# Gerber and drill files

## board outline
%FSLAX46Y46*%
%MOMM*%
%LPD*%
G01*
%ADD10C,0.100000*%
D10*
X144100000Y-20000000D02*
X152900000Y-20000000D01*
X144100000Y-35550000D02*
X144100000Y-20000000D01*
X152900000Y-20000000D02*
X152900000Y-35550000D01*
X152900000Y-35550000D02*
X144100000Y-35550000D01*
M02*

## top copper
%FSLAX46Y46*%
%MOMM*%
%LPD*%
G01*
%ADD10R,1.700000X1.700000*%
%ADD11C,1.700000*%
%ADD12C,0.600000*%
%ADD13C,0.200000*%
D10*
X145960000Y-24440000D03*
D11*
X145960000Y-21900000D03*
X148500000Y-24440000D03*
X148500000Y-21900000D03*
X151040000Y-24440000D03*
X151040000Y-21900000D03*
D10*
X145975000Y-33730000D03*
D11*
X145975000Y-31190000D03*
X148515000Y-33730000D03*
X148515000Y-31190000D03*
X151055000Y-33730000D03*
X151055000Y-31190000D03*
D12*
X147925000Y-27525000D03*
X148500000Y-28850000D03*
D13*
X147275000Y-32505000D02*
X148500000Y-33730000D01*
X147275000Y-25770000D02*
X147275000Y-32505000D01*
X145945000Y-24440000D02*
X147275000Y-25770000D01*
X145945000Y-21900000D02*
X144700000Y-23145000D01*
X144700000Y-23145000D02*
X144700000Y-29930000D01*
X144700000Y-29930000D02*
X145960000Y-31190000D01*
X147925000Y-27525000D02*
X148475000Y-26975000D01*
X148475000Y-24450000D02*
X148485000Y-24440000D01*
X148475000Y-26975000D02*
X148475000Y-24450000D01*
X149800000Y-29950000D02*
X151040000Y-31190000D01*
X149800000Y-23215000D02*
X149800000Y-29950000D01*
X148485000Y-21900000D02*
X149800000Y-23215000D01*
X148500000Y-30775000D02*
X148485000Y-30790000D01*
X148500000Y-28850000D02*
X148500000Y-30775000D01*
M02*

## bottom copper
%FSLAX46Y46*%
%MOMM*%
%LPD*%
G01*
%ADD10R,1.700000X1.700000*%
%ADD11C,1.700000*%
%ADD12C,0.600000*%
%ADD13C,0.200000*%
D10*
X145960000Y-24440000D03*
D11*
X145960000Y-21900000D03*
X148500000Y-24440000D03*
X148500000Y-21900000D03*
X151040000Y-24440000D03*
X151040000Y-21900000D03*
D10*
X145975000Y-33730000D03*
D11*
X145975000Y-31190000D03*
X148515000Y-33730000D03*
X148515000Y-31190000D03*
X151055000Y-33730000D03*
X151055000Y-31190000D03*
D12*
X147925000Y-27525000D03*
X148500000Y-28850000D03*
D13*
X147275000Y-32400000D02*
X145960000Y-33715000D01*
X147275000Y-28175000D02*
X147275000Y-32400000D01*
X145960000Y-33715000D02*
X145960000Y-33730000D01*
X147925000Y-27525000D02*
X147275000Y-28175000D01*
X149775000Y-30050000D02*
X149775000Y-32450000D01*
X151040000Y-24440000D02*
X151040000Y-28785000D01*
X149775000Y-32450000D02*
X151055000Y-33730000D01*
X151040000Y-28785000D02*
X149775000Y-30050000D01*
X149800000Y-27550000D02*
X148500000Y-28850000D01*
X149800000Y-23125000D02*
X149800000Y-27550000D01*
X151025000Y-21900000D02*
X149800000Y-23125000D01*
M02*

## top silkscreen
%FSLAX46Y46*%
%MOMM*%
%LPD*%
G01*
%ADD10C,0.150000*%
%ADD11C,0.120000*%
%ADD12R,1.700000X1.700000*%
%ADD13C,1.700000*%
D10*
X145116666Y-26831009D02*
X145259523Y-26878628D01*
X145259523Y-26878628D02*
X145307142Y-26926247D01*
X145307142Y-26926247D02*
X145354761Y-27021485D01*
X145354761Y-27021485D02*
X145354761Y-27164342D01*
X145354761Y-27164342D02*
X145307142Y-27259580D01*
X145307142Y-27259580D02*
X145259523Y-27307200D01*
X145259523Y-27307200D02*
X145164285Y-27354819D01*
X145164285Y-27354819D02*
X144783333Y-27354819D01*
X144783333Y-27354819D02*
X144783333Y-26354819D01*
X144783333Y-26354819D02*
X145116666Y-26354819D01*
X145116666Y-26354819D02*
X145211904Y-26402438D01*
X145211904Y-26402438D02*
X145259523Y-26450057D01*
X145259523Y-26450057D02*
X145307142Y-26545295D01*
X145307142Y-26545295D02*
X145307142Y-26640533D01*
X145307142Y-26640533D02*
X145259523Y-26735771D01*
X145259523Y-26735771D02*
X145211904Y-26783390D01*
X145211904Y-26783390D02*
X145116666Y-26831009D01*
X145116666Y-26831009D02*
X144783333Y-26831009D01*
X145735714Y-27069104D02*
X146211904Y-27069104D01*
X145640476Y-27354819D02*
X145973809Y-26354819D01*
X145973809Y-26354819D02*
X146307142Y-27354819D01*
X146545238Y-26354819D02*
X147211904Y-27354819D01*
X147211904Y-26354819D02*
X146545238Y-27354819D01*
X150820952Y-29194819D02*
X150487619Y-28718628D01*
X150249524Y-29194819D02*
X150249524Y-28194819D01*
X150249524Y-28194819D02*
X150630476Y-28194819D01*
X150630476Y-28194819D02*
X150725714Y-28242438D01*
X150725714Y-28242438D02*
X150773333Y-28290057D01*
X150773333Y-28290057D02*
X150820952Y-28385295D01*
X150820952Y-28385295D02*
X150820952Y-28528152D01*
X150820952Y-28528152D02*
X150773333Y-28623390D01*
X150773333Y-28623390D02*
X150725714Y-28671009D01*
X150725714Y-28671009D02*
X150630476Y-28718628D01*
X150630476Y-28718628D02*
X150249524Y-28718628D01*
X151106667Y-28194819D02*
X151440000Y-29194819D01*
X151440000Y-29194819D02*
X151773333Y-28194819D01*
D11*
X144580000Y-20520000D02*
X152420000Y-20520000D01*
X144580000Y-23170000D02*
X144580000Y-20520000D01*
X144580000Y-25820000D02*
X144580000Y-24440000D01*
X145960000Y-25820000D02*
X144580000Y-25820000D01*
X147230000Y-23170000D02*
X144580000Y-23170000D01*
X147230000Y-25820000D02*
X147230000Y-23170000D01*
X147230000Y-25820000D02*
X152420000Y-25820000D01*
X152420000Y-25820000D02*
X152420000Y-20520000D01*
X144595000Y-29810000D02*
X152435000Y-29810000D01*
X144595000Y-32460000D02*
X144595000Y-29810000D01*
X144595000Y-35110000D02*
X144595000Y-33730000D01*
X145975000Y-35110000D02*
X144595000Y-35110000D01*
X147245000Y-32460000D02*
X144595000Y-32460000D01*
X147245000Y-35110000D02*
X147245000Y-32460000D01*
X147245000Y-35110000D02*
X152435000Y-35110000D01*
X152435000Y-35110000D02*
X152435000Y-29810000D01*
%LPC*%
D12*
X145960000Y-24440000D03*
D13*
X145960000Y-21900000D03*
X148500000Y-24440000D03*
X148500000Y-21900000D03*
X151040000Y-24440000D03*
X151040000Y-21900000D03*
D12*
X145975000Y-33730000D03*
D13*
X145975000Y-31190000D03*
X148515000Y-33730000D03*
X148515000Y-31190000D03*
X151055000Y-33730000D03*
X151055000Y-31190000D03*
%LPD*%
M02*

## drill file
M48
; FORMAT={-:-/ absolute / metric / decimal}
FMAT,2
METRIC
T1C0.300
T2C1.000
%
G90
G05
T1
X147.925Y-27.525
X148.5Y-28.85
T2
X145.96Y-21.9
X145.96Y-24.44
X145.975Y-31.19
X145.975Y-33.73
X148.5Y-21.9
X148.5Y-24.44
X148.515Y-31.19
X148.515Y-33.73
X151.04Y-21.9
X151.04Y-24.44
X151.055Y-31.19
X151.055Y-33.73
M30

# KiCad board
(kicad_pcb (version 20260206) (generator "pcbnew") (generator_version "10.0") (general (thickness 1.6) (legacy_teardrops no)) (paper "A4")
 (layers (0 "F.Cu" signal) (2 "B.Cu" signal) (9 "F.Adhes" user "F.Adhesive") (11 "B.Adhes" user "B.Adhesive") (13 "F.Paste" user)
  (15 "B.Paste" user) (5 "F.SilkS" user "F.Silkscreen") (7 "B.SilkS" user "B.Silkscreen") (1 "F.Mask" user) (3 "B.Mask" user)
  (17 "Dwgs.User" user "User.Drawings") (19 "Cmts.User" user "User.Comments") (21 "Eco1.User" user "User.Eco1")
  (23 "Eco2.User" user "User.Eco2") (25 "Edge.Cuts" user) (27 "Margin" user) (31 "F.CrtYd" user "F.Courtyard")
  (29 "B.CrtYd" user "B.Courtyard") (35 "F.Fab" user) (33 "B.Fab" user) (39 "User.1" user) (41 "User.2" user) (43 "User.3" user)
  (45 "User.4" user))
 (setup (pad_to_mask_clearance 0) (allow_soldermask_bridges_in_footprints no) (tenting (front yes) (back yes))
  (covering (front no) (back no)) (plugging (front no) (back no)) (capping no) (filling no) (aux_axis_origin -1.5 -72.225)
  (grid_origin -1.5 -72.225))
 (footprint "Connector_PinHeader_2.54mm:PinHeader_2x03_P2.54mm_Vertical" (layer "F.Cu") (at 145.96 24.44 90)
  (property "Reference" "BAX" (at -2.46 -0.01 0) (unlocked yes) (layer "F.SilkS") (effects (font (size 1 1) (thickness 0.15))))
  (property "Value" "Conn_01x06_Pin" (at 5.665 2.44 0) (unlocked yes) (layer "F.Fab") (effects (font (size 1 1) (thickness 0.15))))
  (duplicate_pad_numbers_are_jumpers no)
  (fp_line (start 3.92 -1.38) (end 3.92 6.46) (stroke (width 0.12) (type solid)) (layer "F.SilkS"))
  (fp_line (start 1.27 -1.38) (end 3.92 -1.38) (stroke (width 0.12) (type solid)) (layer "F.SilkS"))
  (fp_line (start -1.38 -1.38) (end 0 -1.38) (stroke (width 0.12) (type solid)) (layer "F.SilkS"))
  (fp_line (start -1.38 0) (end -1.38 -1.38) (stroke (width 0.12) (type solid)) (layer "F.SilkS"))
  (fp_line (start 1.27 1.27) (end 1.27 -1.38) (stroke (width 0.12) (type solid)) (layer "F.SilkS"))
  (fp_line (start -1.38 1.27) (end 1.27 1.27) (stroke (width 0.12) (type solid)) (layer "F.SilkS"))
  (fp_line (start -1.38 1.27) (end -1.38 6.46) (stroke (width 0.12) (type solid)) (layer "F.SilkS"))
  (fp_line (start -1.38 6.46) (end 3.92 6.46) (stroke (width 0.12) (type solid)) (layer "F.SilkS"))
  (pad "1" thru_hole rect (at 0 0 90) (size 1.7 1.7) (drill 1) (layers "*.Cu" "*.Mask") (remove_unused_layers no) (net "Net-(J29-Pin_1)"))
  (pad "2" thru_hole circle (at 2.54 0 90) (size 1.7 1.7) (drill 1) (layers "*.Cu" "*.Mask") (remove_unused_layers no)
   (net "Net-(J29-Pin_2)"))
  (pad "3" thru_hole circle (at 0 2.54 90) (size 1.7 1.7) (drill 1) (layers "*.Cu" "*.Mask") (remove_unused_layers no)
   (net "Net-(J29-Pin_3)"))
  (pad "4" thru_hole circle (at 2.54 2.54 90) (size 1.7 1.7) (drill 1) (layers "*.Cu" "*.Mask") (remove_unused_layers no)
   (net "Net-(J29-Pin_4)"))
  (pad "5" thru_hole circle (at 0 5.08 90) (size 1.7 1.7) (drill 1) (layers "*.Cu" "*.Mask") (remove_unused_layers no)
   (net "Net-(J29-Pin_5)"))
  (pad "6" thru_hole circle (at 2.54 5.08 90) (size 1.7 1.7) (drill 1) (layers "*.Cu" "*.Mask") (remove_unused_layers no)
   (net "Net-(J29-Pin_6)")))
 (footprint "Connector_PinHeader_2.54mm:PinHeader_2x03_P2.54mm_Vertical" (layer "F.Cu") (at 145.975 33.73 90)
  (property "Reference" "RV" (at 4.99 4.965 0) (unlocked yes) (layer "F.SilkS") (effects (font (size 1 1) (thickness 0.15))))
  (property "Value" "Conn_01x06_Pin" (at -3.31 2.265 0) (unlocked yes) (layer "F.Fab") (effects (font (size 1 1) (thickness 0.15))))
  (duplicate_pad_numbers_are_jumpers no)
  (fp_line (start 3.92 -1.38) (end 3.92 6.46) (stroke (width 0.12) (type solid)) (layer "F.SilkS"))
  (fp_line (start 1.27 -1.38) (end 3.92 -1.38) (stroke (width 0.12) (type solid)) (layer "F.SilkS"))
  (fp_line (start -1.38 -1.38) (end 0 -1.38) (stroke (width 0.12) (type solid)) (layer "F.SilkS"))
  (fp_line (start -1.38 0) (end -1.38 -1.38) (stroke (width 0.12) (type solid)) (layer "F.SilkS"))
  (fp_line (start 1.27 1.27) (end 1.27 -1.38) (stroke (width 0.12) (type solid)) (layer "F.SilkS"))
  (fp_line (start -1.38 1.27) (end 1.27 1.27) (stroke (width 0.12) (type solid)) (layer "F.SilkS"))
  (fp_line (start -1.38 1.27) (end -1.38 6.46) (stroke (width 0.12) (type solid)) (layer "F.SilkS"))
  (fp_line (start -1.38 6.46) (end 3.92 6.46) (stroke (width 0.12) (type solid)) (layer "F.SilkS"))
  (pad "1" thru_hole rect (at 0 0 90) (size 1.7 1.7) (drill 1) (layers "*.Cu" "*.Mask") (remove_unused_layers no) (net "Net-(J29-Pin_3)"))
  (pad "2" thru_hole circle (at 2.54 0 90) (size 1.7 1.7) (drill 1) (layers "*.Cu" "*.Mask") (remove_unused_layers no)
   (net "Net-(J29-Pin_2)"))
  (pad "3" thru_hole circle (at 0 2.54 90) (size 1.7 1.7) (drill 1) (layers "*.Cu" "*.Mask") (remove_unused_layers no)
   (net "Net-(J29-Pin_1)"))
  (pad "4" thru_hole circle (at 2.54 2.54 90) (size 1.7 1.7) (drill 1) (layers "*.Cu" "*.Mask") (remove_unused_layers no)
   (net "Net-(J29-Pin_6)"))
  (pad "5" thru_hole circle (at 0 5.08 90) (size 1.7 1.7) (drill 1) (layers "*.Cu" "*.Mask") (remove_unused_layers no)
   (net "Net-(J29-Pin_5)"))
  (pad "6" thru_hole circle (at 2.54 5.08 90) (size 1.7 1.7) (drill 1) (layers "*.Cu" "*.Mask") (remove_unused_layers no)
   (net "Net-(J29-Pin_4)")))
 (gr_line (start 144.1 20) (end 152.9 20) (stroke (width 0.1) (type default)) (layer "Edge.Cuts"))
 (gr_line (start 144.1 35.55) (end 144.1 20) (stroke (width 0.1) (type default)) (layer "Edge.Cuts"))
 (gr_line (start 152.9 20) (end 152.9 35.55) (stroke (width 0.1) (type default)) (layer "Edge.Cuts"))
 (gr_line (start 152.9 35.55) (end 144.1 35.55) (stroke (width 0.1) (type default)) (layer "Edge.Cuts"))
 (segment (start 147.275 32.505) (end 148.5 33.73) (width 0.2) (layer "F.Cu") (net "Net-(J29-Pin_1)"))
 (segment (start 147.275 25.77) (end 147.275 32.505) (width 0.2) (layer "F.Cu") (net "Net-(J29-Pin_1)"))
 (segment (start 145.945 24.44) (end 147.275 25.77) (width 0.2) (layer "F.Cu") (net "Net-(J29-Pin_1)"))
 (segment (start 145.945 21.9) (end 144.7 23.145) (width 0.2) (layer "F.Cu") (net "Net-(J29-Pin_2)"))
 (segment (start 144.7 23.145) (end 144.7 29.93) (width 0.2) (layer "F.Cu") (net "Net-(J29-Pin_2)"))
 (segment (start 144.7 29.93) (end 145.96 31.19) (width 0.2) (layer "F.Cu") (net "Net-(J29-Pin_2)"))
 (segment (start 147.925 27.525) (end 148.475 26.975) (width 0.2) (layer "F.Cu") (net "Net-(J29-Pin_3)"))
 (segment (start 148.475 24.45) (end 148.485 24.44) (width 0.2) (layer "F.Cu") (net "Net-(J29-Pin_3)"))
 (segment (start 148.475 26.975) (end 148.475 24.45) (width 0.2) (layer "F.Cu") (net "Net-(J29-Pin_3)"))
 (via (at 147.925 27.525) (size 0.6) (drill 0.3) (layers "F.Cu" "B.Cu") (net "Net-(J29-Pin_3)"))
 (segment (start 147.275 32.4) (end 145.96 33.715) (width 0.2) (layer "B.Cu") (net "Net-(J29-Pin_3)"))
 (segment (start 147.275 28.175) (end 147.275 32.4) (width 0.2) (layer "B.Cu") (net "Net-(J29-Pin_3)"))
 (segment (start 145.96 33.715) (end 145.96 33.73) (width 0.2) (layer "B.Cu") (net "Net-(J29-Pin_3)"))
 (segment (start 147.925 27.525) (end 147.275 28.175) (width 0.2) (layer "B.Cu") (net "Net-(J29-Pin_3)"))
 (segment (start 149.8 29.95) (end 151.04 31.19) (width 0.2) (layer "F.Cu") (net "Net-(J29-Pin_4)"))
 (segment (start 149.8 23.215) (end 149.8 29.95) (width 0.2) (layer "F.Cu") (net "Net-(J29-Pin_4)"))
 (segment (start 148.485 21.9) (end 149.8 23.215) (width 0.2) (layer "F.Cu") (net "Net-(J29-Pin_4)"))
 (segment (start 149.775 30.05) (end 149.775 32.45) (width 0.2) (layer "B.Cu") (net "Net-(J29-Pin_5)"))
 (segment (start 151.04 24.44) (end 151.04 28.785) (width 0.2) (layer "B.Cu") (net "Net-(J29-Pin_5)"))
 (segment (start 149.775 32.45) (end 151.055 33.73) (width 0.2) (layer "B.Cu") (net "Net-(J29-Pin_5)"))
 (segment (start 151.04 28.785) (end 149.775 30.05) (width 0.2) (layer "B.Cu") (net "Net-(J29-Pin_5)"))
 (segment (start 148.5 30.775) (end 148.485 30.79) (width 0.2) (layer "F.Cu") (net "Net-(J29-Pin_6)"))
 (segment (start 148.5 28.85) (end 148.5 30.775) (width 0.2) (layer "F.Cu") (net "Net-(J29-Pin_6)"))
 (via (at 148.5 28.85) (size 0.6) (drill 0.3) (layers "F.Cu" "B.Cu") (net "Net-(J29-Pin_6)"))
 (segment (start 149.8 27.55) (end 148.5 28.85) (width 0.2) (layer "B.Cu") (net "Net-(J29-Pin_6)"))
 (segment (start 149.8 23.125) (end 149.8 27.55) (width 0.2) (layer "B.Cu") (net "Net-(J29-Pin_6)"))
 (segment (start 151.025 21.9) (end 149.8 23.125) (width 0.2) (layer "B.Cu") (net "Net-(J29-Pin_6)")))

